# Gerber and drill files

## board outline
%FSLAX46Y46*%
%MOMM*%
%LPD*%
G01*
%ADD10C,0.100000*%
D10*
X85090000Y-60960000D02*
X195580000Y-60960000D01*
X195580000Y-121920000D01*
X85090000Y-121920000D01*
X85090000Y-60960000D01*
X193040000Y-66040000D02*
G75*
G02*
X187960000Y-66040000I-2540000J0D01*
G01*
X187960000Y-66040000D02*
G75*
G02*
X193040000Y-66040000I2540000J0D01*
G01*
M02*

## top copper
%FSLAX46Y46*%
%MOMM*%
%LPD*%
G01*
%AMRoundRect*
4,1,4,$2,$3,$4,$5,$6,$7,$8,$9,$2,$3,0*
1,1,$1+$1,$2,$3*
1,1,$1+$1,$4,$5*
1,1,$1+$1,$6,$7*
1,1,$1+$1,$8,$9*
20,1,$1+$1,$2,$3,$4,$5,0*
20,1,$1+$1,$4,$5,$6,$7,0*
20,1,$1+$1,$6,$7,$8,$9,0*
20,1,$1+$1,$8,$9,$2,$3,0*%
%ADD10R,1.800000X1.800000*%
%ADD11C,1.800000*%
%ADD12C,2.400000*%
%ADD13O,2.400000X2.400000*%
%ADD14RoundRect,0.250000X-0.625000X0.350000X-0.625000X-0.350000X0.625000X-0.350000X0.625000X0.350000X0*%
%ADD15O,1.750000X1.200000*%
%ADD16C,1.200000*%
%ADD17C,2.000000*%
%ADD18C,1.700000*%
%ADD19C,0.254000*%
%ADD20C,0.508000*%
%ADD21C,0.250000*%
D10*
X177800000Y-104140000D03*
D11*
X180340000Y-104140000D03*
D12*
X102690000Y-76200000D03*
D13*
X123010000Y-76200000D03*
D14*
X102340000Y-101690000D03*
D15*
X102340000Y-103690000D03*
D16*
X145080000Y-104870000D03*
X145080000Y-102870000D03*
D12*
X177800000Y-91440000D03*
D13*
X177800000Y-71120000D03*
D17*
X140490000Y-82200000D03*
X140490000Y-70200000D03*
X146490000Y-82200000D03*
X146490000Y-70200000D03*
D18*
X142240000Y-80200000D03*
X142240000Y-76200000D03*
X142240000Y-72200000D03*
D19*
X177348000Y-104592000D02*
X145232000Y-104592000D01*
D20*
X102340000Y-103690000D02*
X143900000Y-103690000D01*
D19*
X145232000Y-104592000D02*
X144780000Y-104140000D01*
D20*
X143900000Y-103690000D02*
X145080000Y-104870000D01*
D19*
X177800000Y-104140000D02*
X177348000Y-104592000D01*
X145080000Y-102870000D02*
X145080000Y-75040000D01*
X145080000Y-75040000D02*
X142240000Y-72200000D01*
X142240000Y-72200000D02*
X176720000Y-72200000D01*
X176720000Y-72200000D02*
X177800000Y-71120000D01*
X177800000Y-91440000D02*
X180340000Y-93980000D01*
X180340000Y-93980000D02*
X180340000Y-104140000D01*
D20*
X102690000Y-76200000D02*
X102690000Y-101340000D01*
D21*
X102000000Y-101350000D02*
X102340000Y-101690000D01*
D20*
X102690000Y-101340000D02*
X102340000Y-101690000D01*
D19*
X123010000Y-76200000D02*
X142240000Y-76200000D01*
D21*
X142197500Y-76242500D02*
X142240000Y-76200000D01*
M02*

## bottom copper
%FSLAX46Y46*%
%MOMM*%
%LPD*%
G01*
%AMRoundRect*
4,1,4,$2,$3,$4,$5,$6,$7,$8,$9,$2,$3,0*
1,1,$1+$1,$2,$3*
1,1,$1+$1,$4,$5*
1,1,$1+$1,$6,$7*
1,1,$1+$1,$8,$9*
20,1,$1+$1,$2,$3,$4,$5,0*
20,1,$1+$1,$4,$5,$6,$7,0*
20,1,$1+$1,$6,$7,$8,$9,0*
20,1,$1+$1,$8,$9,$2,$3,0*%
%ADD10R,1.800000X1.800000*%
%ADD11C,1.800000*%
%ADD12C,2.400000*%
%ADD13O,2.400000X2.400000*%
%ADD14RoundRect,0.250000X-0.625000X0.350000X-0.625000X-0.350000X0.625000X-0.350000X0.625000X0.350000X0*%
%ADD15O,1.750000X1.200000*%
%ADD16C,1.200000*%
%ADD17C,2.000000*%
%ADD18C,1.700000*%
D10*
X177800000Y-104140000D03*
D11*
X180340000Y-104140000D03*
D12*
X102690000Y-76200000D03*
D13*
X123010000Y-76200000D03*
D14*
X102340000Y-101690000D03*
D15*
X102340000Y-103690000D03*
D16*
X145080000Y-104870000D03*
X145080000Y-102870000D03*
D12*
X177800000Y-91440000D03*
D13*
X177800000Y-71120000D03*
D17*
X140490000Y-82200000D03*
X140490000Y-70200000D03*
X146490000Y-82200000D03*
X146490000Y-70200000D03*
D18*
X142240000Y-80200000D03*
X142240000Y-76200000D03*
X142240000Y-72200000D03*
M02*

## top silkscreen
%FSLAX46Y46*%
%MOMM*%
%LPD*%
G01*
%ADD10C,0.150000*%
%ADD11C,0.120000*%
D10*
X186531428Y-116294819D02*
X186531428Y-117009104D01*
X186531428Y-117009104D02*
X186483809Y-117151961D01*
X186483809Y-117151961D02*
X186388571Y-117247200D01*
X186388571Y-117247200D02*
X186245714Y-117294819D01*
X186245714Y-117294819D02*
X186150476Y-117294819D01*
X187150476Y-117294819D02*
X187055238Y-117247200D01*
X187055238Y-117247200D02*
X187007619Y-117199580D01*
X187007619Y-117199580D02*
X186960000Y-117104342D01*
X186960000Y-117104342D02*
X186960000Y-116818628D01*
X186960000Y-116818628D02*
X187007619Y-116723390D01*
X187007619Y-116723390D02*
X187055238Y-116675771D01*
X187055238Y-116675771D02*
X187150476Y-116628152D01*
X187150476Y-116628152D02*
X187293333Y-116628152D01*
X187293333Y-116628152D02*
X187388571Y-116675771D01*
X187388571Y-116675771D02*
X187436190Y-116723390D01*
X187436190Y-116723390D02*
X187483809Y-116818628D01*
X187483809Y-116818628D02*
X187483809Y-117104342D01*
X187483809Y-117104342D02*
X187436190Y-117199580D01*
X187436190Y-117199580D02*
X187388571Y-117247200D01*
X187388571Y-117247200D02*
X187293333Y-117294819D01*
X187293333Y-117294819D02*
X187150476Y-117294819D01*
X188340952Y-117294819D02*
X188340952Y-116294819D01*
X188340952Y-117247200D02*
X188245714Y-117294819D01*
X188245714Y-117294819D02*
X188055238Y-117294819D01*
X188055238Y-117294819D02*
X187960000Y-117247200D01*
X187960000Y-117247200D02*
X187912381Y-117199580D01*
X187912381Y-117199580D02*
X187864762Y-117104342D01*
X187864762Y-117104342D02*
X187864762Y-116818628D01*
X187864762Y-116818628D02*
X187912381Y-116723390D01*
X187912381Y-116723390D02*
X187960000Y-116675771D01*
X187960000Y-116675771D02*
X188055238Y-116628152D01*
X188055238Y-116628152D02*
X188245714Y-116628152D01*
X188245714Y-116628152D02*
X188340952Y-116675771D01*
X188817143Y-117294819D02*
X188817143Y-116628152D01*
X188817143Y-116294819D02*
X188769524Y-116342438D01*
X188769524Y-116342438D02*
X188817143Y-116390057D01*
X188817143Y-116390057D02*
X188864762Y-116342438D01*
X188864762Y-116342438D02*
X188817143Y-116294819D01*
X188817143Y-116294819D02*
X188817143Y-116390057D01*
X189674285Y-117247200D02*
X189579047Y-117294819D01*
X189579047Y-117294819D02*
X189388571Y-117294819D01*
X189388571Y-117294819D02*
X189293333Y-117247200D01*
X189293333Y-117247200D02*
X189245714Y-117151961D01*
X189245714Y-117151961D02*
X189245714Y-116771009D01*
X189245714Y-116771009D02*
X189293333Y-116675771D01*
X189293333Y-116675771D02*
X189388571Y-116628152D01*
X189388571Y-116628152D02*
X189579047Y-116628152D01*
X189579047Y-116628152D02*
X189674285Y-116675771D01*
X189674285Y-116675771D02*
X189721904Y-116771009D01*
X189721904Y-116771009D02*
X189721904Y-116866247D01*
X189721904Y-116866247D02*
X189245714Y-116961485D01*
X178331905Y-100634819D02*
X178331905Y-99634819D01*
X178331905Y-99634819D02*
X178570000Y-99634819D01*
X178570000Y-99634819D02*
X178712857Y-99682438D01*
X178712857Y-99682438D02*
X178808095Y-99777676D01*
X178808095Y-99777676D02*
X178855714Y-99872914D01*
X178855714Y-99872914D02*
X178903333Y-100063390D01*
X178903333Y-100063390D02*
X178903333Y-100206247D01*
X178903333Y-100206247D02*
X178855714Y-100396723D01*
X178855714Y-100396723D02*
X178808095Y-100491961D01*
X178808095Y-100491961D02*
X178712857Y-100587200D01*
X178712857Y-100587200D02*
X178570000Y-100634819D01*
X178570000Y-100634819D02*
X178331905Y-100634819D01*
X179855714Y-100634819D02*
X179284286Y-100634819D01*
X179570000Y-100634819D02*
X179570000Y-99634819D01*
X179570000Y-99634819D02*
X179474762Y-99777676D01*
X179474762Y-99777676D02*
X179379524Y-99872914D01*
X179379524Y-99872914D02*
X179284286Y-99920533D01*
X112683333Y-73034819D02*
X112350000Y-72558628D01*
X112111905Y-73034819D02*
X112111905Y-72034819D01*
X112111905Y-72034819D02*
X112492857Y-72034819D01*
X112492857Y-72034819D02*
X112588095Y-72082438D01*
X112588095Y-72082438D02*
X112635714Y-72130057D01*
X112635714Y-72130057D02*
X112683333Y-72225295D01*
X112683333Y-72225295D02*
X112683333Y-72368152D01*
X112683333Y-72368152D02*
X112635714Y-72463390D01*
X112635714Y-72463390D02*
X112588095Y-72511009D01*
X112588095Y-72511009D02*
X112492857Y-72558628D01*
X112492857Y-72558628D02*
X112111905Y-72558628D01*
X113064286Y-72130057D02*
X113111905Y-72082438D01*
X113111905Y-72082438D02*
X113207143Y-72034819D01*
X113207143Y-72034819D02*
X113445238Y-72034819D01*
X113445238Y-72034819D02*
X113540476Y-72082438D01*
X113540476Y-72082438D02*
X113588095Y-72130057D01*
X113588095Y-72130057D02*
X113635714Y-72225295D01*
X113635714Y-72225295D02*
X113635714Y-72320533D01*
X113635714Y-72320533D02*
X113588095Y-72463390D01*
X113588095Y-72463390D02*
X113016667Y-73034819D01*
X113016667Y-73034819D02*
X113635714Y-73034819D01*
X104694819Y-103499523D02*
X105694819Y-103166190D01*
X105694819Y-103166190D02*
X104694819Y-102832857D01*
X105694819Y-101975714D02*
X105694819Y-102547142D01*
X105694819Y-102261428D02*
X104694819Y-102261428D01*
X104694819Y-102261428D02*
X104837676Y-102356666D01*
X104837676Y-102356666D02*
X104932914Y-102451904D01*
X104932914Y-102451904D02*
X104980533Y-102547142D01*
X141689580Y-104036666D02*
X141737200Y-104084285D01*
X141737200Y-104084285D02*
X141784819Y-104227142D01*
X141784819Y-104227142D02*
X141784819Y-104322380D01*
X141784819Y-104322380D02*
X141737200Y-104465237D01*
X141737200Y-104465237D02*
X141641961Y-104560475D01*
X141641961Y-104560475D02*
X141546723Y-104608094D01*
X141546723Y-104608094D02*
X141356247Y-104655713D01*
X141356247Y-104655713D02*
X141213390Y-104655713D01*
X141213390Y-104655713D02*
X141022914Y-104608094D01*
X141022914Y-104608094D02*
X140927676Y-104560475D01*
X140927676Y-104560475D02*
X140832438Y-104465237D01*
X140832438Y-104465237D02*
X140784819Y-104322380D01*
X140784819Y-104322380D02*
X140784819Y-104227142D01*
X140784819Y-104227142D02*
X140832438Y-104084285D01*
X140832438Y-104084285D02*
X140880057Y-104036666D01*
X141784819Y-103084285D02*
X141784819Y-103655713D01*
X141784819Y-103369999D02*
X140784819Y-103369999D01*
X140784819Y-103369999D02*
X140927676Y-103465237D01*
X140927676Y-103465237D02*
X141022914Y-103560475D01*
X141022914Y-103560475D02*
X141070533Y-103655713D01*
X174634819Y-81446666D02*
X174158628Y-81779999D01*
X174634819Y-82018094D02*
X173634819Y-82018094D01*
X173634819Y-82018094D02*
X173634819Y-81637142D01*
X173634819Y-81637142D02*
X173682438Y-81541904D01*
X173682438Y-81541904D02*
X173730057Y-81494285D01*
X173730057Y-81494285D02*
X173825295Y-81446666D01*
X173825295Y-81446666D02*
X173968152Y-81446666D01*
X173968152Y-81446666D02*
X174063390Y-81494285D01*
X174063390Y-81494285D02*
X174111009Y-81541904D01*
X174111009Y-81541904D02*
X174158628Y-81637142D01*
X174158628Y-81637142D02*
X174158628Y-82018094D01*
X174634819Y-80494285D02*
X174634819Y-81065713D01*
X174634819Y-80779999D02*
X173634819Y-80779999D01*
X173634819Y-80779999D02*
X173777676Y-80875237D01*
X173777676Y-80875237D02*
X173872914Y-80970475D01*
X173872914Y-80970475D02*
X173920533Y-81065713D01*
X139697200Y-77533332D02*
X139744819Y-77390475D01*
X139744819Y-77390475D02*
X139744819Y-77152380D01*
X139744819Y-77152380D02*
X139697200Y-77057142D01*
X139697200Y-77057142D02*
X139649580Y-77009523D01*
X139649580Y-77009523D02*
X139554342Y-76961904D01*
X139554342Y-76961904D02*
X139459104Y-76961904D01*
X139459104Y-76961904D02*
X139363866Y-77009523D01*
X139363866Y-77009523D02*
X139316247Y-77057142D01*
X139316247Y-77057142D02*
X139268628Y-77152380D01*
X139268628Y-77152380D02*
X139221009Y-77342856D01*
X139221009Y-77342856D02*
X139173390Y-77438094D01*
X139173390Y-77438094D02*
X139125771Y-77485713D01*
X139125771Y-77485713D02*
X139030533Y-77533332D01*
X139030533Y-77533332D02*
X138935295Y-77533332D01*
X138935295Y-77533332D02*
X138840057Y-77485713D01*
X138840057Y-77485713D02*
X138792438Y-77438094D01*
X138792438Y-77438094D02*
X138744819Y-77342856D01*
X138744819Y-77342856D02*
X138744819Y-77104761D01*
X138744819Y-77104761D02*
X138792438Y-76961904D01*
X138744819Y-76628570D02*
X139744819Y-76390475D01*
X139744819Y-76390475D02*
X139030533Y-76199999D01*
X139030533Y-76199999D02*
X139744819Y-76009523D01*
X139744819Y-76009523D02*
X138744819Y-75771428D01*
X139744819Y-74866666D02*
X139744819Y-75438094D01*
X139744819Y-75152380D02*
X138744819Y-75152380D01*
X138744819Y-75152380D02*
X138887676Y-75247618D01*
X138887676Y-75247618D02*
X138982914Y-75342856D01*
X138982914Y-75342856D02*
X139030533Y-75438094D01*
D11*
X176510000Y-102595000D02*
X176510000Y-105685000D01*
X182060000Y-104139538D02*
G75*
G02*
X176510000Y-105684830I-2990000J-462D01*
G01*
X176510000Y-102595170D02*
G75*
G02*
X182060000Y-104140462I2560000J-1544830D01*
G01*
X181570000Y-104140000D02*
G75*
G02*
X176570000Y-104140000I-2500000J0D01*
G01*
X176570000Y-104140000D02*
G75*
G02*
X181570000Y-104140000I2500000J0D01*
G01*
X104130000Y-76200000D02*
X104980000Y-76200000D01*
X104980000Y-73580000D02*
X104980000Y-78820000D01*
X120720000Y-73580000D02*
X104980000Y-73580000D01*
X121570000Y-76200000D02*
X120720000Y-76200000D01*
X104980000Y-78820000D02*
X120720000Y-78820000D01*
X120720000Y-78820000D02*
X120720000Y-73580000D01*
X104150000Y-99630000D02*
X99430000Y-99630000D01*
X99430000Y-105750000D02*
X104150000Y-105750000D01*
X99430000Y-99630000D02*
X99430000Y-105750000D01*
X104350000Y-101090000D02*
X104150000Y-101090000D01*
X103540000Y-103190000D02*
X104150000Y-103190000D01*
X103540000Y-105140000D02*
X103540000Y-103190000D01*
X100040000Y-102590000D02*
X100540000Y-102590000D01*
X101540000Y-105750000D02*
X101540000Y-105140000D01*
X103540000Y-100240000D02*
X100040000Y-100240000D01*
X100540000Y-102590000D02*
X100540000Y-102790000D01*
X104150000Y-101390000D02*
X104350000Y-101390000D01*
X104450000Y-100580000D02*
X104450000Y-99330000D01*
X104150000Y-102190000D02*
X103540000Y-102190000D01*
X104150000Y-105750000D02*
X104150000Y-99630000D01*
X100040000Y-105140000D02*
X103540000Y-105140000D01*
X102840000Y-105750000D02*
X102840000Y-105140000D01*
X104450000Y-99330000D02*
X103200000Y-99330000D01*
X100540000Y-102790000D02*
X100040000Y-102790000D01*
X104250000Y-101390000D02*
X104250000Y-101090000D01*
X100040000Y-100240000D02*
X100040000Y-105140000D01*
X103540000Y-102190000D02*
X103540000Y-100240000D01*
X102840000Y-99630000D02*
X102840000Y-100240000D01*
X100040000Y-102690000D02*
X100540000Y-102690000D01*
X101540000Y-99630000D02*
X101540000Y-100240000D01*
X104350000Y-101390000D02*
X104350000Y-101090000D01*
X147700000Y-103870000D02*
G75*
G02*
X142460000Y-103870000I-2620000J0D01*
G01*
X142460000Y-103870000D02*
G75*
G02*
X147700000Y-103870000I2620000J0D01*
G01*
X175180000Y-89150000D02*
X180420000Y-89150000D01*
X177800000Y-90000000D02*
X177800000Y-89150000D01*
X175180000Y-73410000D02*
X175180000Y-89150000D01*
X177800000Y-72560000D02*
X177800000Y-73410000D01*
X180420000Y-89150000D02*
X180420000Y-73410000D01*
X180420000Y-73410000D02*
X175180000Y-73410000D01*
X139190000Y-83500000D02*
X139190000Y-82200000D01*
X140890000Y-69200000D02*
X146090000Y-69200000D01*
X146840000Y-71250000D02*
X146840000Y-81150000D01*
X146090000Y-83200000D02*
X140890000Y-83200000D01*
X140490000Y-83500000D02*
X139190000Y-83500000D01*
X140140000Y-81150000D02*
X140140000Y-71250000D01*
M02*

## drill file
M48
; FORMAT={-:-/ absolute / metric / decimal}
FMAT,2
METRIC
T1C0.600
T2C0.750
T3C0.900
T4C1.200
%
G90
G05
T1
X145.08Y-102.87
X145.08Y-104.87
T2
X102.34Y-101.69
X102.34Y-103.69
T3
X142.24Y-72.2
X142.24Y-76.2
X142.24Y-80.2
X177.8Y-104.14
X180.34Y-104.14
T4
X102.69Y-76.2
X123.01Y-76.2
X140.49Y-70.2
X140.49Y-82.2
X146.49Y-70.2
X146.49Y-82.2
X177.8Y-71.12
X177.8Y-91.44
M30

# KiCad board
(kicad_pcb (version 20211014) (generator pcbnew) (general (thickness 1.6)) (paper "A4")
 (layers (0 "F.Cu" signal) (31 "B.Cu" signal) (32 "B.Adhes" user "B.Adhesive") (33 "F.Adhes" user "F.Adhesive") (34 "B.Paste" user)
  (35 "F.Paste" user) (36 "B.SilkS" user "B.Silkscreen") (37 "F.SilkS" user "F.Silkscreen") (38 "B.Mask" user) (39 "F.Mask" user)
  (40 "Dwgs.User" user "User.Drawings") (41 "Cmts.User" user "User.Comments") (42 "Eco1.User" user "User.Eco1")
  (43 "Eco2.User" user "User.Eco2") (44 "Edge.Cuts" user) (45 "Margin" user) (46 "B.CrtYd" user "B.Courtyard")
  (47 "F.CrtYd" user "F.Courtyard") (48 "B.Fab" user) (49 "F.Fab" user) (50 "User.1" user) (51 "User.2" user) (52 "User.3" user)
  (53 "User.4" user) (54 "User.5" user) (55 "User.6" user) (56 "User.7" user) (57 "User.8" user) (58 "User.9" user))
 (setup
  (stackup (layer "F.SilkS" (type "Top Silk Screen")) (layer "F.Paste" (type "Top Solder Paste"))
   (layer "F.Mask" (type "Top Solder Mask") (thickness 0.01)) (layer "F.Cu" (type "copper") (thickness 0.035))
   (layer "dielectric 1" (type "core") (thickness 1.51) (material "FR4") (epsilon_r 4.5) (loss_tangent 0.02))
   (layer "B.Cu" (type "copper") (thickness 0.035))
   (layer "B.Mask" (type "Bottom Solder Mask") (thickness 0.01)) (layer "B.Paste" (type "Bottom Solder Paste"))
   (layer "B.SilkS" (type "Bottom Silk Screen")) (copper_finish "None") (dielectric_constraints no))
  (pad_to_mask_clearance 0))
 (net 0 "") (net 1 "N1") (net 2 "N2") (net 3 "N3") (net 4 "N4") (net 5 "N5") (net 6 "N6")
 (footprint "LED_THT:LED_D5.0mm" (layer "F.Cu") (at 177.8 104.14)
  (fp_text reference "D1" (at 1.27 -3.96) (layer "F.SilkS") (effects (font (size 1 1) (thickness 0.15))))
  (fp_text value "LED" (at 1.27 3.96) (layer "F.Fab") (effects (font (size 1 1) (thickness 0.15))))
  (fp_line (start -1.29 -1.545) (end -1.29 1.545) (layer "F.SilkS") (width 0.12))
  (fp_arc (start 4.26 -0.000462) (mid 2.072002 2.880433) (end -1.29 1.54483) (layer "F.SilkS") (width 0.12))
  (fp_arc (start -1.29 -1.54483) (mid 2.072002 -2.880433) (end 4.26 0.000462) (layer "F.SilkS") (width 0.12))
  (fp_circle (center 1.27 0) (end 3.77 0) (layer "F.SilkS") (width 0.12) (fill none))
  (pad "1" thru_hole rect (at 0 0) (size 1.8 1.8) (drill 0.9) (layers *.Cu *.Mask) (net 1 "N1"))
  (pad "2" thru_hole circle (at 2.54 0) (size 1.8 1.8) (drill 0.9) (layers *.Cu *.Mask) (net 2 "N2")))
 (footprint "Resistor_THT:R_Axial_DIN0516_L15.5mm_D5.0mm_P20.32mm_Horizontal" (layer "F.Cu") (at 102.69 76.2)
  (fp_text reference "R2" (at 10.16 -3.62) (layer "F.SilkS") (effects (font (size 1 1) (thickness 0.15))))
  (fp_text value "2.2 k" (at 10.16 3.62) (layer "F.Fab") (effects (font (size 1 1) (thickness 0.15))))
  (fp_line (start 1.44 0) (end 2.29 0) (layer "F.SilkS") (width 0.12))
  (fp_line (start 2.29 -2.62) (end 2.29 2.62) (layer "F.SilkS") (width 0.12))
  (fp_line (start 18.03 -2.62) (end 2.29 -2.62) (layer "F.SilkS") (width 0.12))
  (fp_line (start 18.88 0) (end 18.03 0) (layer "F.SilkS") (width 0.12))
  (fp_line (start 2.29 2.62) (end 18.03 2.62) (layer "F.SilkS") (width 0.12))
  (fp_line (start 18.03 2.62) (end 18.03 -2.62) (layer "F.SilkS") (width 0.12))
  (pad "1" thru_hole circle (at 0 0) (size 2.4 2.4) (drill 1.2) (layers *.Cu *.Mask) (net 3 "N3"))
  (pad "2" thru_hole oval (at 20.32 0) (size 2.4 2.4) (drill 1.2) (layers *.Cu *.Mask) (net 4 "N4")))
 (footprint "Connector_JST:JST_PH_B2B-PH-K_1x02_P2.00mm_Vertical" (layer "F.Cu") (at 102.34 101.69 -90)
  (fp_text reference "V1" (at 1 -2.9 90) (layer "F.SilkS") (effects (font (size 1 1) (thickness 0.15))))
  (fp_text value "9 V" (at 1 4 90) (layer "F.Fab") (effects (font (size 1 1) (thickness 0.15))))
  (fp_line (start -2.06 -1.81) (end -2.06 2.91) (layer "F.SilkS") (width 0.12))
  (fp_line (start 4.06 2.91) (end 4.06 -1.81) (layer "F.SilkS") (width 0.12))
  (fp_line (start -2.06 2.91) (end 4.06 2.91) (layer "F.SilkS") (width 0.12))
  (fp_line (start -0.6 -2.01) (end -0.6 -1.81) (layer "F.SilkS") (width 0.12))
  (fp_line (start 1.5 -1.2) (end 1.5 -1.81) (layer "F.SilkS") (width 0.12))
  (fp_line (start 3.45 -1.2) (end 1.5 -1.2) (layer "F.SilkS") (width 0.12))
  (fp_line (start 0.9 2.3) (end 0.9 1.8) (layer "F.SilkS") (width 0.12))
  (fp_line (start 4.06 0.8) (end 3.45 0.8) (layer "F.SilkS") (width 0.12))
  (fp_line (start -1.45 -1.2) (end -1.45 2.3) (layer "F.SilkS") (width 0.12))
  (fp_line (start 0.9 1.8) (end 1.1 1.8) (layer "F.SilkS") (width 0.12))
  (fp_line (start -0.3 -1.81) (end -0.3 -2.01) (layer "F.SilkS") (width 0.12))
  (fp_line (start -1.11 -2.11) (end -2.36 -2.11) (layer "F.SilkS") (width 0.12))
  (fp_line (start 0.5 -1.81) (end 0.5 -1.2) (layer "F.SilkS") (width 0.12))
  (fp_line (start 4.06 -1.81) (end -2.06 -1.81) (layer "F.SilkS") (width 0.12))
  (fp_line (start 3.45 2.3) (end 3.45 -1.2) (layer "F.SilkS") (width 0.12))
  (fp_line (start 4.06 -0.5) (end 3.45 -0.5) (layer "F.SilkS") (width 0.12))
  (fp_line (start -2.36 -2.11) (end -2.36 -0.86) (layer "F.SilkS") (width 0.12))
  (fp_line (start 1.1 1.8) (end 1.1 2.3) (layer "F.SilkS") (width 0.12))
  (fp_line (start -0.3 -1.91) (end -0.6 -1.91) (layer "F.SilkS") (width 0.12))
  (fp_line (start -1.45 2.3) (end 3.45 2.3) (layer "F.SilkS") (width 0.12))
  (fp_line (start 0.5 -1.2) (end -1.45 -1.2) (layer "F.SilkS") (width 0.12))
  (fp_line (start -2.06 -0.5) (end -1.45 -0.5) (layer "F.SilkS") (width 0.12))
  (fp_line (start 1 2.3) (end 1 1.8) (layer "F.SilkS") (width 0.12))
  (fp_line (start -2.06 0.8) (end -1.45 0.8) (layer "F.SilkS") (width 0.12))
  (fp_line (start -0.3 -2.01) (end -0.6 -2.01) (layer "F.SilkS") (width 0.12))
  (pad "1" thru_hole roundrect (at 0 0 270) (size 1.2 1.75) (drill 0.75) (layers *.Cu *.Mask) (roundrect_rratio 0.208333) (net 3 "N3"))
  (pad "2" thru_hole oval (at 2 0 270) (size 1.2 1.75) (drill 0.75) (layers *.Cu *.Mask) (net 1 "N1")))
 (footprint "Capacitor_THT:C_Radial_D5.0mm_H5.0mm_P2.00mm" (layer "F.Cu") (at 145.08 104.87 90)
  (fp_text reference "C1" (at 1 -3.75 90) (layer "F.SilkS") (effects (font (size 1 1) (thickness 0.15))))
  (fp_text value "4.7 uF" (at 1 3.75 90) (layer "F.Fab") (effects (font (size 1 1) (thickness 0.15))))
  (fp_circle (center 1 0) (end 3.62 0) (layer "F.SilkS") (width 0.12) (fill none))
  (pad "1" thru_hole circle (at 0 0 90) (size 1.2 1.2) (drill 0.6) (layers *.Cu *.Mask) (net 1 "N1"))
  (pad "2" thru_hole circle (at 2 0 90) (size 1.2 1.2) (drill 0.6) (layers *.Cu *.Mask) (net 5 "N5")))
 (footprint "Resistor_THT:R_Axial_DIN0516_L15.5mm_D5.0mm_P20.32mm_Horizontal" (layer "F.Cu") (at 177.8 91.44 90)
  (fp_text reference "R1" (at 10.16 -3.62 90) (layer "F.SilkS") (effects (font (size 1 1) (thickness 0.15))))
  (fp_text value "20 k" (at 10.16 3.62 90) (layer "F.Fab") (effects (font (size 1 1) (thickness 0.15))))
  (fp_line (start 2.29 -2.62) (end 2.29 2.62) (layer "F.SilkS") (width 0.12))
  (fp_line (start 1.44 0) (end 2.29 0) (layer "F.SilkS") (width 0.12))
  (fp_line (start 18.03 -2.62) (end 2.29 -2.62) (layer "F.SilkS") (width 0.12))
  (fp_line (start 18.88 0) (end 18.03 0) (layer "F.SilkS") (width 0.12))
  (fp_line (start 2.29 2.62) (end 18.03 2.62) (layer "F.SilkS") (width 0.12))
  (fp_line (start 18.03 2.62) (end 18.03 -2.62) (layer "F.SilkS") (width 0.12))
  (pad "1" thru_hole circle (at 0 0 90) (size 2.4 2.4) (drill 1.2) (layers *.Cu *.Mask) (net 2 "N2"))
  (pad "2" thru_hole oval (at 20.32 0 90) (size 2.4 2.4) (drill 1.2) (layers *.Cu *.Mask) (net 5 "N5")))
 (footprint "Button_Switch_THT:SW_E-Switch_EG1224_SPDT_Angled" (layer "F.Cu") (at 142.24 80.2 90)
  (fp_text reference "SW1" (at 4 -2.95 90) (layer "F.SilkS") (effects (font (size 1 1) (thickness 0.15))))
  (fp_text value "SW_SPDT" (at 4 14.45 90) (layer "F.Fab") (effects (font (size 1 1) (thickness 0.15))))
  (fp_line (start -3.3 -3.05) (end -2 -3.05) (layer "F.SilkS") (width 0.12))
  (fp_line (start 11 -1.35) (end 11 3.85) (layer "F.SilkS") (width 0.12))
  (fp_line (start 8.95 4.6) (end -0.95 4.6) (layer "F.SilkS") (width 0.12))
  (fp_line (start -3 3.85) (end -3 -1.35) (layer "F.SilkS") (width 0.12))
  (fp_line (start -3.3 -1.75) (end -3.3 -3.05) (layer "F.SilkS") (width 0.12))
  (fp_line (start -0.95 -2.1) (end 8.95 -2.1) (layer "F.SilkS") (width 0.12))
  (pad "" thru_hole circle (at -2 -1.75 90) (size 2 2) (drill 1.2) (layers *.Cu *.Mask))
  (pad "" thru_hole circle (at 10 -1.75 90) (size 2 2) (drill 1.2) (layers *.Cu *.Mask))
  (pad "" thru_hole circle (at -2 4.25 90) (size 2 2) (drill 1.2) (layers *.Cu *.Mask))
  (pad "" thru_hole circle (at 10 4.25 90) (size 2 2) (drill 1.2) (layers *.Cu *.Mask))
  (pad "1" thru_hole circle (at 0 0 90) (size 1.7 1.7) (drill 0.9) (layers *.Cu *.Mask) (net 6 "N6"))
  (pad "2" thru_hole circle (at 4 0 90) (size 1.7 1.7) (drill 0.9) (layers *.Cu *.Mask) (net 4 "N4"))
  (pad "3" thru_hole circle (at 8 0 90) (size 1.7 1.7) (drill 0.9) (layers *.Cu *.Mask) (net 5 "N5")))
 (gr_rect (start 85.09 60.96) (end 195.58 121.92) (layer "Edge.Cuts") (width 0.1) (fill none))
 (gr_circle (center 190.5 66.04) (end 193.04 66.04) (layer "Edge.Cuts") (width 0.1) (fill none))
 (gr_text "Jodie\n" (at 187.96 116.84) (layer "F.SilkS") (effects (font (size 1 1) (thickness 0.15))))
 (segment (start 177.348 104.592) (end 145.232 104.592) (width 0.254) (layer "F.Cu") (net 1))
 (segment (start 102.34 103.69) (end 143.9 103.69) (width 0.508) (layer "F.Cu") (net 1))
 (segment (start 145.232 104.592) (end 144.78 104.14) (width 0.254) (layer "F.Cu") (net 1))
 (segment (start 143.9 103.69) (end 145.08 104.87) (width 0.508) (layer "F.Cu") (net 1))
 (segment (start 177.8 104.14) (end 177.348 104.592) (width 0.254) (layer "F.Cu") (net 1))
 (segment (start 145.08 102.87) (end 145.08 75.04) (width 0.254) (layer "F.Cu") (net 5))
 (segment (start 145.08 75.04) (end 142.24 72.2) (width 0.254) (layer "F.Cu") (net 5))
 (segment (start 142.24 72.2) (end 176.72 72.2) (width 0.254) (layer "F.Cu") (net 5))
 (segment (start 176.72 72.2) (end 177.8 71.12) (width 0.254) (layer "F.Cu") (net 5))
 (segment (start 177.8 91.44) (end 180.34 93.98) (width 0.254) (layer "F.Cu") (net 2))
 (segment (start 180.34 93.98) (end 180.34 104.14) (width 0.254) (layer "F.Cu") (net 2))
 (segment (start 102.69 76.2) (end 102.69 101.34) (width 0.508) (layer "F.Cu") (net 3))
 (segment (start 102 101.35) (end 102.34 101.69) (width 0.25) (layer "F.Cu") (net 3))
 (segment (start 102.69 101.34) (end 102.34 101.69) (width 0.508) (layer "F.Cu") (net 3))
 (segment (start 123.01 76.2) (end 142.24 76.2) (width 0.254) (layer "F.Cu") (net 4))
 (segment (start 142.1975 76.2425) (end 142.24 76.2) (width 0.25) (layer "F.Cu") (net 4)))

